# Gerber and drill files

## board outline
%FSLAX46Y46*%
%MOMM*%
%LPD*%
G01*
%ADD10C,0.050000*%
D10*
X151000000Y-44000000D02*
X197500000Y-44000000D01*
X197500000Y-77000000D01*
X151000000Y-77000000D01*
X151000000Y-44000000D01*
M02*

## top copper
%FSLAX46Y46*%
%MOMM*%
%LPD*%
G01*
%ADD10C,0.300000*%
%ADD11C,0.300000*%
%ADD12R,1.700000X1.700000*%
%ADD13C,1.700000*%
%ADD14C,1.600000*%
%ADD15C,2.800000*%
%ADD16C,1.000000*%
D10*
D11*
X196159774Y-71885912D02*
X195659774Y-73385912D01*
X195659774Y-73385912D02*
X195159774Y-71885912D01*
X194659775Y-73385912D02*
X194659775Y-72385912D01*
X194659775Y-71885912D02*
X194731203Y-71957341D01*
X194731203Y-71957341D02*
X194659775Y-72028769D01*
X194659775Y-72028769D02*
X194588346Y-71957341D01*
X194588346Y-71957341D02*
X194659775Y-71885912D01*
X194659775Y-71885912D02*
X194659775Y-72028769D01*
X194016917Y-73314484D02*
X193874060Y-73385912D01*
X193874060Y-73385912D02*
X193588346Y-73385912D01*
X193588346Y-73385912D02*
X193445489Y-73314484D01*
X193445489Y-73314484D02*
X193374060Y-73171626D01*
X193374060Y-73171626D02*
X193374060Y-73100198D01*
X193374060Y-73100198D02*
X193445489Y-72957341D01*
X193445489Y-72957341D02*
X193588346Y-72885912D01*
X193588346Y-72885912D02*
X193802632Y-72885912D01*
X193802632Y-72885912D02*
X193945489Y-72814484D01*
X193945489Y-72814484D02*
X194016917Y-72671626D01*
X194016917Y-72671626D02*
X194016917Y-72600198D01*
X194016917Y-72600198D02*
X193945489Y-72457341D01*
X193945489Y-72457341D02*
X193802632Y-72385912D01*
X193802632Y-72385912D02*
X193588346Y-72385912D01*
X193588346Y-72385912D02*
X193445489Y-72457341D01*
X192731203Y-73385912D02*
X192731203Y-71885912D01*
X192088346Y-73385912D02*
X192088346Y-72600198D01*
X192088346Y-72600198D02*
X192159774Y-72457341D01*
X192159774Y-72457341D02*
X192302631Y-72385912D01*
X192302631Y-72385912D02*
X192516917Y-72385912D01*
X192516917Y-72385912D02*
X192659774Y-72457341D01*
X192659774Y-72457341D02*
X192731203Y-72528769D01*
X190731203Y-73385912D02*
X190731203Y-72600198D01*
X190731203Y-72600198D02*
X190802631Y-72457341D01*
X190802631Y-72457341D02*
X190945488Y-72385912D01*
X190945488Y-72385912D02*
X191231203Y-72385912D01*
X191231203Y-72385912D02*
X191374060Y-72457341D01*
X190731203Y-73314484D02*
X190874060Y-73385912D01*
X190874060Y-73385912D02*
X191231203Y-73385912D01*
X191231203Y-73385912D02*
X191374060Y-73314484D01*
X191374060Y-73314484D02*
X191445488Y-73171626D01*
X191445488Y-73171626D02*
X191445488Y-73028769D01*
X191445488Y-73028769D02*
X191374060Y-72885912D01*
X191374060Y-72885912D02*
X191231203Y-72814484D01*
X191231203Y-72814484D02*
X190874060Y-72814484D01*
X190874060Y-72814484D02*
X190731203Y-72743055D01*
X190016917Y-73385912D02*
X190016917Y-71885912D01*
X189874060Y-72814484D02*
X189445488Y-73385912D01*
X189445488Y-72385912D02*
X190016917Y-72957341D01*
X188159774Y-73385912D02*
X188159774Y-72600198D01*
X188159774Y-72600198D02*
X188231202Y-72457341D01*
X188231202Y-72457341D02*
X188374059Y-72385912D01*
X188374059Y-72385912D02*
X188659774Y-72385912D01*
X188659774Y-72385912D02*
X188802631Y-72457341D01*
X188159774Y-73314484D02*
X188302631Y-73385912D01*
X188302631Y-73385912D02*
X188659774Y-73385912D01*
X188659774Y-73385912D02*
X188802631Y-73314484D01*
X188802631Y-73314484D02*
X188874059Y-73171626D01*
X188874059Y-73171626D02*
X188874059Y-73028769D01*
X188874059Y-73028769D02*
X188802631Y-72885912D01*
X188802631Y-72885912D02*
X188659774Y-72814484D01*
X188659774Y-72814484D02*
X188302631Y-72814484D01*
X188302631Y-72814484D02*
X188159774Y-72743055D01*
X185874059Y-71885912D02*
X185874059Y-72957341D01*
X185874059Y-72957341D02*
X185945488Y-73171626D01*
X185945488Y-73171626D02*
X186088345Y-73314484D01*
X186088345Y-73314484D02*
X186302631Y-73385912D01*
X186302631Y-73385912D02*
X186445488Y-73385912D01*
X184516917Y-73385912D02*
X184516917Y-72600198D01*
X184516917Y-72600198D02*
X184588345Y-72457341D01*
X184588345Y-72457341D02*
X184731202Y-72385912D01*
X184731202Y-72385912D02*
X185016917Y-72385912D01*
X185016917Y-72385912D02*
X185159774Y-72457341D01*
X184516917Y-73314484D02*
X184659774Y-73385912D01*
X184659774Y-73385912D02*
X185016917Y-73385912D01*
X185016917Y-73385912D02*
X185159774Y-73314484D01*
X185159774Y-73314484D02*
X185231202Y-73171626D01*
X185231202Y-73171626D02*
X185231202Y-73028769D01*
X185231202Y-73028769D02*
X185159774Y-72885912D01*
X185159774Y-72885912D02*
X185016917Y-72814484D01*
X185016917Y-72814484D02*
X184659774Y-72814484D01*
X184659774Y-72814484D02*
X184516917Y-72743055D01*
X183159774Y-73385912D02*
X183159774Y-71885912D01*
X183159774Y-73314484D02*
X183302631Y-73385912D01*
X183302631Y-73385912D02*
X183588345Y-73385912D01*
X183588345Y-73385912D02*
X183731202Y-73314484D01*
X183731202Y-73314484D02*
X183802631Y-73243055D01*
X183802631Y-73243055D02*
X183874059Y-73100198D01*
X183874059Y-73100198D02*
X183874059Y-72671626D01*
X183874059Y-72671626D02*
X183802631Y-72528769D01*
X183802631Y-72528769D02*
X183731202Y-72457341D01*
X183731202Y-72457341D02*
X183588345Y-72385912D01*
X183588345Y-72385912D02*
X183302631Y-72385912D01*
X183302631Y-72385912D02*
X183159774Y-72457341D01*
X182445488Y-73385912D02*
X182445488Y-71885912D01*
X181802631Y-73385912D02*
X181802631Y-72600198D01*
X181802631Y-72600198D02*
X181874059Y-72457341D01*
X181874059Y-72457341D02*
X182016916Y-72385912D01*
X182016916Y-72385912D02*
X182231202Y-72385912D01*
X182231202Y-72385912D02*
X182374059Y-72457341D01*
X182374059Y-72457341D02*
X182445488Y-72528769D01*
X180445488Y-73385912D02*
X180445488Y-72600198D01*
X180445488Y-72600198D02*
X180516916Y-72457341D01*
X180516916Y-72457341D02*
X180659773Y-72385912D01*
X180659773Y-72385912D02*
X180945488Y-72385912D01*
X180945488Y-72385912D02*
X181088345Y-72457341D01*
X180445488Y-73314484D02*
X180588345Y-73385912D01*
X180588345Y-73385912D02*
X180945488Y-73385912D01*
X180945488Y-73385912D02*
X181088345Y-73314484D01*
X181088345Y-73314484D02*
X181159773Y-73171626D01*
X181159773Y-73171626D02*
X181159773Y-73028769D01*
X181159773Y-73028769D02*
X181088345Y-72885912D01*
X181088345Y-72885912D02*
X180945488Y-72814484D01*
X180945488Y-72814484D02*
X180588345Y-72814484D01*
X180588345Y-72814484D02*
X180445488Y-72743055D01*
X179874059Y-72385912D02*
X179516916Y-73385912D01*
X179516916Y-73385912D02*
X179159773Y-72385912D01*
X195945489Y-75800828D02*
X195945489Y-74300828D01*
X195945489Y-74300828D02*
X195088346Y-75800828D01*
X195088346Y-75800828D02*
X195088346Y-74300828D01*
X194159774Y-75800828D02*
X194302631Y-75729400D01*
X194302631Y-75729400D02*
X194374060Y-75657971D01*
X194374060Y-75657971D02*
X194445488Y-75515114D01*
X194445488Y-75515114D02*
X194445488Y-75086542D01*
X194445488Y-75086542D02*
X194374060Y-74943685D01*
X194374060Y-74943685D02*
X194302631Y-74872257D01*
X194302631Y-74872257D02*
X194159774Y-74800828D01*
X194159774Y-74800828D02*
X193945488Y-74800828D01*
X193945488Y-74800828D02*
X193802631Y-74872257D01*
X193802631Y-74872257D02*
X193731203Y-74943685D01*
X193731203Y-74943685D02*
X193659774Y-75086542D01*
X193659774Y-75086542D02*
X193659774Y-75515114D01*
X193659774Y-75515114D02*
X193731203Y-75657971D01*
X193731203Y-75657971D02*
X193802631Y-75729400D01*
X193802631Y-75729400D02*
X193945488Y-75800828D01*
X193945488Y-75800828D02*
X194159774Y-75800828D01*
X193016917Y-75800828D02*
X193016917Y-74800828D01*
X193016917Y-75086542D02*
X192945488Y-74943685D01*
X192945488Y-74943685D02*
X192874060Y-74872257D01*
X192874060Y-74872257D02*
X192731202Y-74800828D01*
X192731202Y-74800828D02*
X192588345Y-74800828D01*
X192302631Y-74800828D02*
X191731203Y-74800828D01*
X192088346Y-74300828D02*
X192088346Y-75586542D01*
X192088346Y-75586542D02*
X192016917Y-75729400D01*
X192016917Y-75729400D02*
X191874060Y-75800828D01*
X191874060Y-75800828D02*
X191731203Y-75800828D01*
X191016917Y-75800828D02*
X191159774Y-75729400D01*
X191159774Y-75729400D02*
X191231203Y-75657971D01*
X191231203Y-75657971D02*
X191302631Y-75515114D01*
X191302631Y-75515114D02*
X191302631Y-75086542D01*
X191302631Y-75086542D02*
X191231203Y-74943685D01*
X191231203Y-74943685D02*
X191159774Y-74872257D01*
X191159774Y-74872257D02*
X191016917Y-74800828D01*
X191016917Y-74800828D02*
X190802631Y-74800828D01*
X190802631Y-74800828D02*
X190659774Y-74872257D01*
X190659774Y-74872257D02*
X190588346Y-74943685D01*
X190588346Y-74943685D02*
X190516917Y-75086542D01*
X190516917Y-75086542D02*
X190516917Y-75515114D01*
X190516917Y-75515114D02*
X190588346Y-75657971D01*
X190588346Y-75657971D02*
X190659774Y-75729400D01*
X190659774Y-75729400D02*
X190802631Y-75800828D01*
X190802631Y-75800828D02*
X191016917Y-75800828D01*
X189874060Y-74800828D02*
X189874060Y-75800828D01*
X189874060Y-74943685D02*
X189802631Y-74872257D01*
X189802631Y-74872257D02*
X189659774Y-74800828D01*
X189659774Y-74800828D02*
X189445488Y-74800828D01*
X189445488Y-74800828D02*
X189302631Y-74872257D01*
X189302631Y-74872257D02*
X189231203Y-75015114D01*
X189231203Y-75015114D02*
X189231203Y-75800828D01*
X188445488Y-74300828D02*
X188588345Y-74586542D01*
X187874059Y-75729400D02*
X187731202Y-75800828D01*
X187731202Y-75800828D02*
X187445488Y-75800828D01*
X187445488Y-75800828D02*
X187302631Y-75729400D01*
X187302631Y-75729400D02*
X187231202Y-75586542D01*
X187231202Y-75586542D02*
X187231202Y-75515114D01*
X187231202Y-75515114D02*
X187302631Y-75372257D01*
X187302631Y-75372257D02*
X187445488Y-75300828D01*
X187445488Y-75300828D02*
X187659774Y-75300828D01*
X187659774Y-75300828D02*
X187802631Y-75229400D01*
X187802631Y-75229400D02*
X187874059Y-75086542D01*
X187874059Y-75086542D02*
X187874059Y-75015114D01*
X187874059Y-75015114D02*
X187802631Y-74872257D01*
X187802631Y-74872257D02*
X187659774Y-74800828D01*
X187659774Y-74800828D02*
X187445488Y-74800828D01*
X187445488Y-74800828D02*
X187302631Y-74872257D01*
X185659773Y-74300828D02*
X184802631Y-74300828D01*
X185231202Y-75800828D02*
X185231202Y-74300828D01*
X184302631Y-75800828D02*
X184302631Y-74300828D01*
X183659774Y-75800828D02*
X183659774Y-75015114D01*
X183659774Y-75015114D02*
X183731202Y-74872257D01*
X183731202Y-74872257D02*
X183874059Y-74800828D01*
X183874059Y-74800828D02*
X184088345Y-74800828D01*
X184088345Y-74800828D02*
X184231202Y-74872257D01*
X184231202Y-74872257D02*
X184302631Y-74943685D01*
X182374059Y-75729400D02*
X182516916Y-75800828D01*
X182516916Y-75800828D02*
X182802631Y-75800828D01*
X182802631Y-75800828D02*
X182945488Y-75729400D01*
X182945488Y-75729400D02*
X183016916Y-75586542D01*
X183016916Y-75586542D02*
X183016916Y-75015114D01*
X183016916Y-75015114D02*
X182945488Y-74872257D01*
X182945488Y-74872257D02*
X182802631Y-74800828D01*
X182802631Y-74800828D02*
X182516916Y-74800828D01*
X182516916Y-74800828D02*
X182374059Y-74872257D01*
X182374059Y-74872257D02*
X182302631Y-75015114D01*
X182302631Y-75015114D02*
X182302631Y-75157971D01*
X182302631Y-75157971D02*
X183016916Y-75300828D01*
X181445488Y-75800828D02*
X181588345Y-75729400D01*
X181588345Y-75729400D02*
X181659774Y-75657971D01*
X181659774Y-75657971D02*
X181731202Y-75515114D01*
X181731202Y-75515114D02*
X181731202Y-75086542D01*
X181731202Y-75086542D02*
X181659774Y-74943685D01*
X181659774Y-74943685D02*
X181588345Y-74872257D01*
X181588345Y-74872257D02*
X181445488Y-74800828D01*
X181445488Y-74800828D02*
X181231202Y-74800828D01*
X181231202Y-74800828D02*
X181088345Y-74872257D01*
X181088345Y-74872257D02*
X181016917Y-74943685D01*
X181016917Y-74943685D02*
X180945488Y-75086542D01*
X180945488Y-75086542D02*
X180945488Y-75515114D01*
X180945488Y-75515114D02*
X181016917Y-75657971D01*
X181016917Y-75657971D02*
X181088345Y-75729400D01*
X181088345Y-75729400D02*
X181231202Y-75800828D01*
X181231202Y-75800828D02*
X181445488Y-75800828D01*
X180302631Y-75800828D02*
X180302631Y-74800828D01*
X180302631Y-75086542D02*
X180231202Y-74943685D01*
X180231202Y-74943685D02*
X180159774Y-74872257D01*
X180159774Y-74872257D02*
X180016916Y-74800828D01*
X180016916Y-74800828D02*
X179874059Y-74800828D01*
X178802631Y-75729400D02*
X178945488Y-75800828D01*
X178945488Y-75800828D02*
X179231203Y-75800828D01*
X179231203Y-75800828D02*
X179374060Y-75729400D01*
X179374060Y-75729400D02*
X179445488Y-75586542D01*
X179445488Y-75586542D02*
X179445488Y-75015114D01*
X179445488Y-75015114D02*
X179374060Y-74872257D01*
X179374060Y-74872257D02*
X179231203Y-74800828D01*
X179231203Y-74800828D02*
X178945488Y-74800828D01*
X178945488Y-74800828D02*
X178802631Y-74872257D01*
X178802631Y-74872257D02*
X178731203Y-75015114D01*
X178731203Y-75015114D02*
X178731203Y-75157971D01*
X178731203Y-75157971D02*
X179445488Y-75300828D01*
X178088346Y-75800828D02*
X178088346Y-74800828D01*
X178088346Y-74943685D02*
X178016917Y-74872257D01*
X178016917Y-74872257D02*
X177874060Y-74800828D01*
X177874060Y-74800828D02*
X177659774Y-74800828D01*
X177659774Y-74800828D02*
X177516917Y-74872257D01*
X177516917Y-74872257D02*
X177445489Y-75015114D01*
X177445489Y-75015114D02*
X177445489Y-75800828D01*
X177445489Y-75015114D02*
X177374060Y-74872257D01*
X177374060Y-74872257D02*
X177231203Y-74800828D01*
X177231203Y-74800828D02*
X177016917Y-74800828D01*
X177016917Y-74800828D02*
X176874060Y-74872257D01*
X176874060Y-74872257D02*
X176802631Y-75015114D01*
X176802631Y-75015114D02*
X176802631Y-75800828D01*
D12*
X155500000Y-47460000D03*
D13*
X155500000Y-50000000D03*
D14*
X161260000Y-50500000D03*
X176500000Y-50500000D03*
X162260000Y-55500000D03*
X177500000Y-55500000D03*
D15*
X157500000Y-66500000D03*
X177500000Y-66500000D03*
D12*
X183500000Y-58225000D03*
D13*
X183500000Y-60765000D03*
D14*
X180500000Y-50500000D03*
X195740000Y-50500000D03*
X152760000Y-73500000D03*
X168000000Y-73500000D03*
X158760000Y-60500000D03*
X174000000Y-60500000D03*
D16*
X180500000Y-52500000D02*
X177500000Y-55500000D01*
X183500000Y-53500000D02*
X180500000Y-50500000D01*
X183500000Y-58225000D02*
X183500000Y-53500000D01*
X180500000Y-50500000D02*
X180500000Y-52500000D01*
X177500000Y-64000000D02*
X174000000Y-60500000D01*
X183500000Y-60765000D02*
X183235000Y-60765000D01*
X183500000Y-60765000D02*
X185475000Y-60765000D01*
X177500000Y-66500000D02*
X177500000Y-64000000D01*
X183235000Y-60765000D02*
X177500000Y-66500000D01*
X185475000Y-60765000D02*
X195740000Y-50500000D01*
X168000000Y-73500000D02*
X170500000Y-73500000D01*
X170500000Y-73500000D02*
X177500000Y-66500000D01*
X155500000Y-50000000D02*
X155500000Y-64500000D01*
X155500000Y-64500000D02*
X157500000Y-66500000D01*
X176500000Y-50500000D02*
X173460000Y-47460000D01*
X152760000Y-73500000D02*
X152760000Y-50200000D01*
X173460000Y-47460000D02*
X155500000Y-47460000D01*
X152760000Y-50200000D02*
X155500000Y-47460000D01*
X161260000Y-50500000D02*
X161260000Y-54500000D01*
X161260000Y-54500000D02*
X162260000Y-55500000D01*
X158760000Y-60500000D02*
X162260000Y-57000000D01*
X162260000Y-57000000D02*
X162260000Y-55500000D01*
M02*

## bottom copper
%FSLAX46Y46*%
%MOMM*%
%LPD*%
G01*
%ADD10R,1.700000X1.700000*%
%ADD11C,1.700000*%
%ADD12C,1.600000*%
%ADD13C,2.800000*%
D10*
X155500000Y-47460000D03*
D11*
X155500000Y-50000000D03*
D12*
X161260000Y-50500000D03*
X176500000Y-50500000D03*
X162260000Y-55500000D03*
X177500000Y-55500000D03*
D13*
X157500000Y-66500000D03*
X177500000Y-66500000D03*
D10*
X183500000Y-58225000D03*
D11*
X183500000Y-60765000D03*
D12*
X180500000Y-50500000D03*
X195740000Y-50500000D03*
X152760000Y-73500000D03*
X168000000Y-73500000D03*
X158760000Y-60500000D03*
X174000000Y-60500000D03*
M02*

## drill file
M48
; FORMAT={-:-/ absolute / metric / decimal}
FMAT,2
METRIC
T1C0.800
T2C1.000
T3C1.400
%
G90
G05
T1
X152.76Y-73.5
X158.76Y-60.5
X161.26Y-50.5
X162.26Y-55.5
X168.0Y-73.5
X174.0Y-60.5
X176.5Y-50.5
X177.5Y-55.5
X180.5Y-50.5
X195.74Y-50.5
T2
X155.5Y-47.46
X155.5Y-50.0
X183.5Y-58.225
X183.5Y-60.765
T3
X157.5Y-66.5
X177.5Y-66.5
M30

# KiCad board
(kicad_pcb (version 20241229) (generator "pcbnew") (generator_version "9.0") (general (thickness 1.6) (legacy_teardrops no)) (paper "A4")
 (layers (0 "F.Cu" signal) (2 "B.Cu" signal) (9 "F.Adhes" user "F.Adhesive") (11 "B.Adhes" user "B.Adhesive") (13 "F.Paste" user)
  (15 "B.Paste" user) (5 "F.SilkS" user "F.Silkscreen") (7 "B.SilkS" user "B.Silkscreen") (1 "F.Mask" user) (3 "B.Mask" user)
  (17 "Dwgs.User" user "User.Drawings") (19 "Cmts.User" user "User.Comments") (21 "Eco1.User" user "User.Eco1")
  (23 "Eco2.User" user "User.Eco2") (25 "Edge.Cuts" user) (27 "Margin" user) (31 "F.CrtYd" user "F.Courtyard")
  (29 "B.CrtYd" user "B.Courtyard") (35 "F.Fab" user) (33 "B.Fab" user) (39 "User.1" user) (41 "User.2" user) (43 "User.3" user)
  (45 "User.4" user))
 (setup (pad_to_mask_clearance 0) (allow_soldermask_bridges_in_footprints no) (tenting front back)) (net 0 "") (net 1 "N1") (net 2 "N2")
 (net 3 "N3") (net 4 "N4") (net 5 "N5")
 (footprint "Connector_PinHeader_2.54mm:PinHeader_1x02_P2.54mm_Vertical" (layer "F.Cu") (at 155.5 47.46)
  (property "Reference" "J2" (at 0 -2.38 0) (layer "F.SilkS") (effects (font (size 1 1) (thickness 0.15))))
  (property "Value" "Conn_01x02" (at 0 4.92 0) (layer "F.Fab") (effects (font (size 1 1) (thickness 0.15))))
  (pad "1" thru_hole rect (at 0 0) (size 1.7 1.7) (drill 1) (layers "*.Cu" "*.Mask") (remove_unused_layers no) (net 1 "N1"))
  (pad "2" thru_hole circle (at 0 2.54) (size 1.7 1.7) (drill 1) (layers "*.Cu" "*.Mask") (remove_unused_layers no) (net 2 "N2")))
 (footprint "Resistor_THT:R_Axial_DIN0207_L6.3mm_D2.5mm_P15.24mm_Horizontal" (layer "F.Cu") (at 161.26 50.5)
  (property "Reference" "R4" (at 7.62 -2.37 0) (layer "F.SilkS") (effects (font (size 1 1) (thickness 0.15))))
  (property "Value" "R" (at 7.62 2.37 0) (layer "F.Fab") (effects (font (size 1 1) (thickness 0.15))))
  (pad "1" thru_hole circle (at 0 0) (size 1.6 1.6) (drill 0.8) (layers "*.Cu" "*.Mask") (remove_unused_layers no) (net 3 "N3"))
  (pad "2" thru_hole circle (at 15.24 0) (size 1.6 1.6) (drill 0.8) (layers "*.Cu" "*.Mask") (remove_unused_layers no) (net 1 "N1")))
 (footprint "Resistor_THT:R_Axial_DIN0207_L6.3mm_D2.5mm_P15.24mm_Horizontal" (layer "F.Cu") (at 162.26 55.5)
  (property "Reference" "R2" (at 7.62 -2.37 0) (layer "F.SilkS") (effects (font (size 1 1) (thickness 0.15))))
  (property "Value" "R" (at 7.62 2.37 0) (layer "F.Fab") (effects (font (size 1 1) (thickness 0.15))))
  (pad "1" thru_hole circle (at 0 0) (size 1.6 1.6) (drill 0.8) (layers "*.Cu" "*.Mask") (remove_unused_layers no) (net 3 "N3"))
  (pad "2" thru_hole circle (at 15.24 0) (size 1.6 1.6) (drill 0.8) (layers "*.Cu" "*.Mask") (remove_unused_layers no) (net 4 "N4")))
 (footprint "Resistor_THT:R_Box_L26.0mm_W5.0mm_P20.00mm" (layer "F.Cu") (at 157.5 66.5)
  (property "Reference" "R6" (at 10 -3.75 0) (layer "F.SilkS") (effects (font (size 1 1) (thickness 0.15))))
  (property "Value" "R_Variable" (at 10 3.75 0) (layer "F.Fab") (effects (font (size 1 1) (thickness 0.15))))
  (pad "1" thru_hole circle (at 0 0) (size 2.8 2.8) (drill 1.4) (layers "*.Cu" "*.Mask") (remove_unused_layers no) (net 2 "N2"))
  (pad "2" thru_hole circle (at 20 0) (size 2.8 2.8) (drill 1.4) (layers "*.Cu" "*.Mask") (remove_unused_layers no) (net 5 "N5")))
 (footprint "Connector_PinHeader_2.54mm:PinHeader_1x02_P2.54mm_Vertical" (layer "F.Cu") (at 183.5 58.225)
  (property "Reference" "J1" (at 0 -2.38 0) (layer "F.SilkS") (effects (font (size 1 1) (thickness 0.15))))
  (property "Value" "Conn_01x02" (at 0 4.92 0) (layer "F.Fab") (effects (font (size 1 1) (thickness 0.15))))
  (pad "1" thru_hole rect (at 0 0) (size 1.7 1.7) (drill 1) (layers "*.Cu" "*.Mask") (remove_unused_layers no) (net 4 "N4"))
  (pad "2" thru_hole circle (at 0 2.54) (size 1.7 1.7) (drill 1) (layers "*.Cu" "*.Mask") (remove_unused_layers no) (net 5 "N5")))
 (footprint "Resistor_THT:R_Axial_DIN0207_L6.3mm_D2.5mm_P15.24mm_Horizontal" (layer "F.Cu") (at 180.5 50.5)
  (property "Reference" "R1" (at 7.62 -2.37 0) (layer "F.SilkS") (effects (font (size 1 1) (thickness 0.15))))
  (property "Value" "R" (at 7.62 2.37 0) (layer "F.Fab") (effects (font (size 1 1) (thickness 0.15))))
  (pad "1" thru_hole circle (at 0 0) (size 1.6 1.6) (drill 0.8) (layers "*.Cu" "*.Mask") (remove_unused_layers no) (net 4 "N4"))
  (pad "2" thru_hole circle (at 15.24 0) (size 1.6 1.6) (drill 0.8) (layers "*.Cu" "*.Mask") (remove_unused_layers no) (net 5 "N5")))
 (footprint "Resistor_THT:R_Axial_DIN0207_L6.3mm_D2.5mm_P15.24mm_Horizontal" (layer "F.Cu") (at 152.76 73.5)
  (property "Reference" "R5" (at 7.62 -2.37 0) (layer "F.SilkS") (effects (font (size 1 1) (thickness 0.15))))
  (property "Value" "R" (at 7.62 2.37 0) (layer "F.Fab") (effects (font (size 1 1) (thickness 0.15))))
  (pad "1" thru_hole circle (at 0 0) (size 1.6 1.6) (drill 0.8) (layers "*.Cu" "*.Mask") (remove_unused_layers no) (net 1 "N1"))
  (pad "2" thru_hole circle (at 15.24 0) (size 1.6 1.6) (drill 0.8) (layers "*.Cu" "*.Mask") (remove_unused_layers no) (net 5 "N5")))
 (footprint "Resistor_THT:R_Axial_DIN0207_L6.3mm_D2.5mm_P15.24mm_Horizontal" (layer "F.Cu") (at 158.76 60.5)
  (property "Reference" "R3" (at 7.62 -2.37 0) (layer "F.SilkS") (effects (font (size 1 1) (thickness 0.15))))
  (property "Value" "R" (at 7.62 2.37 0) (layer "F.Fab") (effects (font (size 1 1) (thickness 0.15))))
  (pad "1" thru_hole circle (at 0 0) (size 1.6 1.6) (drill 0.8) (layers "*.Cu" "*.Mask") (remove_unused_layers no) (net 3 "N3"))
  (pad "2" thru_hole circle (at 15.24 0) (size 1.6 1.6) (drill 0.8) (layers "*.Cu" "*.Mask") (remove_unused_layers no) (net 5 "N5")))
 (gr_rect (start 151 44) (end 197.5 77) (stroke (width 0.05) (type default)) (fill no) (layer "Edge.Cuts"))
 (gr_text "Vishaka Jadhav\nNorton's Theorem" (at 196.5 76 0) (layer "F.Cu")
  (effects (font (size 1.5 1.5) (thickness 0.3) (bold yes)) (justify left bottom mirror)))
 (segment (start 180.5 52.5) (end 177.5 55.5) (width 1) (layer "F.Cu") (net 4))
 (segment (start 183.5 53.5) (end 180.5 50.5) (width 1) (layer "F.Cu") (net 4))
 (segment (start 183.5 58.225) (end 183.5 53.5) (width 1) (layer "F.Cu") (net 4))
 (segment (start 180.5 50.5) (end 180.5 52.5) (width 1) (layer "F.Cu") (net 4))
 (segment (start 177.5 64) (end 174 60.5) (width 1) (layer "F.Cu") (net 5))
 (segment (start 183.5 60.765) (end 183.235 60.765) (width 1) (layer "F.Cu") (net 5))
 (segment (start 183.5 60.765) (end 185.475 60.765) (width 1) (layer "F.Cu") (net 5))
 (segment (start 177.5 66.5) (end 177.5 64) (width 1) (layer "F.Cu") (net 5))
 (segment (start 183.235 60.765) (end 177.5 66.5) (width 1) (layer "F.Cu") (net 5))
 (segment (start 185.475 60.765) (end 195.74 50.5) (width 1) (layer "F.Cu") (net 5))
 (segment (start 168 73.5) (end 170.5 73.5) (width 1) (layer "F.Cu") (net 5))
 (segment (start 170.5 73.5) (end 177.5 66.5) (width 1) (layer "F.Cu") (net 5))
 (segment (start 155.5 50) (end 155.5 64.5) (width 1) (layer "F.Cu") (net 2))
 (segment (start 155.5 64.5) (end 157.5 66.5) (width 1) (layer "F.Cu") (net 2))
 (segment (start 176.5 50.5) (end 173.46 47.46) (width 1) (layer "F.Cu") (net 1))
 (segment (start 152.76 73.5) (end 152.76 50.2) (width 1) (layer "F.Cu") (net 1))
 (segment (start 173.46 47.46) (end 155.5 47.46) (width 1) (layer "F.Cu") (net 1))
 (segment (start 152.76 50.2) (end 155.5 47.46) (width 1) (layer "F.Cu") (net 1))
 (segment (start 161.26 50.5) (end 161.26 54.5) (width 1) (layer "F.Cu") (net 3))
 (segment (start 161.26 54.5) (end 162.26 55.5) (width 1) (layer "F.Cu") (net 3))
 (segment (start 158.76 60.5) (end 162.26 57) (width 1) (layer "F.Cu") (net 3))
 (segment (start 162.26 57) (end 162.26 55.5) (width 1) (layer "F.Cu") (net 3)))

